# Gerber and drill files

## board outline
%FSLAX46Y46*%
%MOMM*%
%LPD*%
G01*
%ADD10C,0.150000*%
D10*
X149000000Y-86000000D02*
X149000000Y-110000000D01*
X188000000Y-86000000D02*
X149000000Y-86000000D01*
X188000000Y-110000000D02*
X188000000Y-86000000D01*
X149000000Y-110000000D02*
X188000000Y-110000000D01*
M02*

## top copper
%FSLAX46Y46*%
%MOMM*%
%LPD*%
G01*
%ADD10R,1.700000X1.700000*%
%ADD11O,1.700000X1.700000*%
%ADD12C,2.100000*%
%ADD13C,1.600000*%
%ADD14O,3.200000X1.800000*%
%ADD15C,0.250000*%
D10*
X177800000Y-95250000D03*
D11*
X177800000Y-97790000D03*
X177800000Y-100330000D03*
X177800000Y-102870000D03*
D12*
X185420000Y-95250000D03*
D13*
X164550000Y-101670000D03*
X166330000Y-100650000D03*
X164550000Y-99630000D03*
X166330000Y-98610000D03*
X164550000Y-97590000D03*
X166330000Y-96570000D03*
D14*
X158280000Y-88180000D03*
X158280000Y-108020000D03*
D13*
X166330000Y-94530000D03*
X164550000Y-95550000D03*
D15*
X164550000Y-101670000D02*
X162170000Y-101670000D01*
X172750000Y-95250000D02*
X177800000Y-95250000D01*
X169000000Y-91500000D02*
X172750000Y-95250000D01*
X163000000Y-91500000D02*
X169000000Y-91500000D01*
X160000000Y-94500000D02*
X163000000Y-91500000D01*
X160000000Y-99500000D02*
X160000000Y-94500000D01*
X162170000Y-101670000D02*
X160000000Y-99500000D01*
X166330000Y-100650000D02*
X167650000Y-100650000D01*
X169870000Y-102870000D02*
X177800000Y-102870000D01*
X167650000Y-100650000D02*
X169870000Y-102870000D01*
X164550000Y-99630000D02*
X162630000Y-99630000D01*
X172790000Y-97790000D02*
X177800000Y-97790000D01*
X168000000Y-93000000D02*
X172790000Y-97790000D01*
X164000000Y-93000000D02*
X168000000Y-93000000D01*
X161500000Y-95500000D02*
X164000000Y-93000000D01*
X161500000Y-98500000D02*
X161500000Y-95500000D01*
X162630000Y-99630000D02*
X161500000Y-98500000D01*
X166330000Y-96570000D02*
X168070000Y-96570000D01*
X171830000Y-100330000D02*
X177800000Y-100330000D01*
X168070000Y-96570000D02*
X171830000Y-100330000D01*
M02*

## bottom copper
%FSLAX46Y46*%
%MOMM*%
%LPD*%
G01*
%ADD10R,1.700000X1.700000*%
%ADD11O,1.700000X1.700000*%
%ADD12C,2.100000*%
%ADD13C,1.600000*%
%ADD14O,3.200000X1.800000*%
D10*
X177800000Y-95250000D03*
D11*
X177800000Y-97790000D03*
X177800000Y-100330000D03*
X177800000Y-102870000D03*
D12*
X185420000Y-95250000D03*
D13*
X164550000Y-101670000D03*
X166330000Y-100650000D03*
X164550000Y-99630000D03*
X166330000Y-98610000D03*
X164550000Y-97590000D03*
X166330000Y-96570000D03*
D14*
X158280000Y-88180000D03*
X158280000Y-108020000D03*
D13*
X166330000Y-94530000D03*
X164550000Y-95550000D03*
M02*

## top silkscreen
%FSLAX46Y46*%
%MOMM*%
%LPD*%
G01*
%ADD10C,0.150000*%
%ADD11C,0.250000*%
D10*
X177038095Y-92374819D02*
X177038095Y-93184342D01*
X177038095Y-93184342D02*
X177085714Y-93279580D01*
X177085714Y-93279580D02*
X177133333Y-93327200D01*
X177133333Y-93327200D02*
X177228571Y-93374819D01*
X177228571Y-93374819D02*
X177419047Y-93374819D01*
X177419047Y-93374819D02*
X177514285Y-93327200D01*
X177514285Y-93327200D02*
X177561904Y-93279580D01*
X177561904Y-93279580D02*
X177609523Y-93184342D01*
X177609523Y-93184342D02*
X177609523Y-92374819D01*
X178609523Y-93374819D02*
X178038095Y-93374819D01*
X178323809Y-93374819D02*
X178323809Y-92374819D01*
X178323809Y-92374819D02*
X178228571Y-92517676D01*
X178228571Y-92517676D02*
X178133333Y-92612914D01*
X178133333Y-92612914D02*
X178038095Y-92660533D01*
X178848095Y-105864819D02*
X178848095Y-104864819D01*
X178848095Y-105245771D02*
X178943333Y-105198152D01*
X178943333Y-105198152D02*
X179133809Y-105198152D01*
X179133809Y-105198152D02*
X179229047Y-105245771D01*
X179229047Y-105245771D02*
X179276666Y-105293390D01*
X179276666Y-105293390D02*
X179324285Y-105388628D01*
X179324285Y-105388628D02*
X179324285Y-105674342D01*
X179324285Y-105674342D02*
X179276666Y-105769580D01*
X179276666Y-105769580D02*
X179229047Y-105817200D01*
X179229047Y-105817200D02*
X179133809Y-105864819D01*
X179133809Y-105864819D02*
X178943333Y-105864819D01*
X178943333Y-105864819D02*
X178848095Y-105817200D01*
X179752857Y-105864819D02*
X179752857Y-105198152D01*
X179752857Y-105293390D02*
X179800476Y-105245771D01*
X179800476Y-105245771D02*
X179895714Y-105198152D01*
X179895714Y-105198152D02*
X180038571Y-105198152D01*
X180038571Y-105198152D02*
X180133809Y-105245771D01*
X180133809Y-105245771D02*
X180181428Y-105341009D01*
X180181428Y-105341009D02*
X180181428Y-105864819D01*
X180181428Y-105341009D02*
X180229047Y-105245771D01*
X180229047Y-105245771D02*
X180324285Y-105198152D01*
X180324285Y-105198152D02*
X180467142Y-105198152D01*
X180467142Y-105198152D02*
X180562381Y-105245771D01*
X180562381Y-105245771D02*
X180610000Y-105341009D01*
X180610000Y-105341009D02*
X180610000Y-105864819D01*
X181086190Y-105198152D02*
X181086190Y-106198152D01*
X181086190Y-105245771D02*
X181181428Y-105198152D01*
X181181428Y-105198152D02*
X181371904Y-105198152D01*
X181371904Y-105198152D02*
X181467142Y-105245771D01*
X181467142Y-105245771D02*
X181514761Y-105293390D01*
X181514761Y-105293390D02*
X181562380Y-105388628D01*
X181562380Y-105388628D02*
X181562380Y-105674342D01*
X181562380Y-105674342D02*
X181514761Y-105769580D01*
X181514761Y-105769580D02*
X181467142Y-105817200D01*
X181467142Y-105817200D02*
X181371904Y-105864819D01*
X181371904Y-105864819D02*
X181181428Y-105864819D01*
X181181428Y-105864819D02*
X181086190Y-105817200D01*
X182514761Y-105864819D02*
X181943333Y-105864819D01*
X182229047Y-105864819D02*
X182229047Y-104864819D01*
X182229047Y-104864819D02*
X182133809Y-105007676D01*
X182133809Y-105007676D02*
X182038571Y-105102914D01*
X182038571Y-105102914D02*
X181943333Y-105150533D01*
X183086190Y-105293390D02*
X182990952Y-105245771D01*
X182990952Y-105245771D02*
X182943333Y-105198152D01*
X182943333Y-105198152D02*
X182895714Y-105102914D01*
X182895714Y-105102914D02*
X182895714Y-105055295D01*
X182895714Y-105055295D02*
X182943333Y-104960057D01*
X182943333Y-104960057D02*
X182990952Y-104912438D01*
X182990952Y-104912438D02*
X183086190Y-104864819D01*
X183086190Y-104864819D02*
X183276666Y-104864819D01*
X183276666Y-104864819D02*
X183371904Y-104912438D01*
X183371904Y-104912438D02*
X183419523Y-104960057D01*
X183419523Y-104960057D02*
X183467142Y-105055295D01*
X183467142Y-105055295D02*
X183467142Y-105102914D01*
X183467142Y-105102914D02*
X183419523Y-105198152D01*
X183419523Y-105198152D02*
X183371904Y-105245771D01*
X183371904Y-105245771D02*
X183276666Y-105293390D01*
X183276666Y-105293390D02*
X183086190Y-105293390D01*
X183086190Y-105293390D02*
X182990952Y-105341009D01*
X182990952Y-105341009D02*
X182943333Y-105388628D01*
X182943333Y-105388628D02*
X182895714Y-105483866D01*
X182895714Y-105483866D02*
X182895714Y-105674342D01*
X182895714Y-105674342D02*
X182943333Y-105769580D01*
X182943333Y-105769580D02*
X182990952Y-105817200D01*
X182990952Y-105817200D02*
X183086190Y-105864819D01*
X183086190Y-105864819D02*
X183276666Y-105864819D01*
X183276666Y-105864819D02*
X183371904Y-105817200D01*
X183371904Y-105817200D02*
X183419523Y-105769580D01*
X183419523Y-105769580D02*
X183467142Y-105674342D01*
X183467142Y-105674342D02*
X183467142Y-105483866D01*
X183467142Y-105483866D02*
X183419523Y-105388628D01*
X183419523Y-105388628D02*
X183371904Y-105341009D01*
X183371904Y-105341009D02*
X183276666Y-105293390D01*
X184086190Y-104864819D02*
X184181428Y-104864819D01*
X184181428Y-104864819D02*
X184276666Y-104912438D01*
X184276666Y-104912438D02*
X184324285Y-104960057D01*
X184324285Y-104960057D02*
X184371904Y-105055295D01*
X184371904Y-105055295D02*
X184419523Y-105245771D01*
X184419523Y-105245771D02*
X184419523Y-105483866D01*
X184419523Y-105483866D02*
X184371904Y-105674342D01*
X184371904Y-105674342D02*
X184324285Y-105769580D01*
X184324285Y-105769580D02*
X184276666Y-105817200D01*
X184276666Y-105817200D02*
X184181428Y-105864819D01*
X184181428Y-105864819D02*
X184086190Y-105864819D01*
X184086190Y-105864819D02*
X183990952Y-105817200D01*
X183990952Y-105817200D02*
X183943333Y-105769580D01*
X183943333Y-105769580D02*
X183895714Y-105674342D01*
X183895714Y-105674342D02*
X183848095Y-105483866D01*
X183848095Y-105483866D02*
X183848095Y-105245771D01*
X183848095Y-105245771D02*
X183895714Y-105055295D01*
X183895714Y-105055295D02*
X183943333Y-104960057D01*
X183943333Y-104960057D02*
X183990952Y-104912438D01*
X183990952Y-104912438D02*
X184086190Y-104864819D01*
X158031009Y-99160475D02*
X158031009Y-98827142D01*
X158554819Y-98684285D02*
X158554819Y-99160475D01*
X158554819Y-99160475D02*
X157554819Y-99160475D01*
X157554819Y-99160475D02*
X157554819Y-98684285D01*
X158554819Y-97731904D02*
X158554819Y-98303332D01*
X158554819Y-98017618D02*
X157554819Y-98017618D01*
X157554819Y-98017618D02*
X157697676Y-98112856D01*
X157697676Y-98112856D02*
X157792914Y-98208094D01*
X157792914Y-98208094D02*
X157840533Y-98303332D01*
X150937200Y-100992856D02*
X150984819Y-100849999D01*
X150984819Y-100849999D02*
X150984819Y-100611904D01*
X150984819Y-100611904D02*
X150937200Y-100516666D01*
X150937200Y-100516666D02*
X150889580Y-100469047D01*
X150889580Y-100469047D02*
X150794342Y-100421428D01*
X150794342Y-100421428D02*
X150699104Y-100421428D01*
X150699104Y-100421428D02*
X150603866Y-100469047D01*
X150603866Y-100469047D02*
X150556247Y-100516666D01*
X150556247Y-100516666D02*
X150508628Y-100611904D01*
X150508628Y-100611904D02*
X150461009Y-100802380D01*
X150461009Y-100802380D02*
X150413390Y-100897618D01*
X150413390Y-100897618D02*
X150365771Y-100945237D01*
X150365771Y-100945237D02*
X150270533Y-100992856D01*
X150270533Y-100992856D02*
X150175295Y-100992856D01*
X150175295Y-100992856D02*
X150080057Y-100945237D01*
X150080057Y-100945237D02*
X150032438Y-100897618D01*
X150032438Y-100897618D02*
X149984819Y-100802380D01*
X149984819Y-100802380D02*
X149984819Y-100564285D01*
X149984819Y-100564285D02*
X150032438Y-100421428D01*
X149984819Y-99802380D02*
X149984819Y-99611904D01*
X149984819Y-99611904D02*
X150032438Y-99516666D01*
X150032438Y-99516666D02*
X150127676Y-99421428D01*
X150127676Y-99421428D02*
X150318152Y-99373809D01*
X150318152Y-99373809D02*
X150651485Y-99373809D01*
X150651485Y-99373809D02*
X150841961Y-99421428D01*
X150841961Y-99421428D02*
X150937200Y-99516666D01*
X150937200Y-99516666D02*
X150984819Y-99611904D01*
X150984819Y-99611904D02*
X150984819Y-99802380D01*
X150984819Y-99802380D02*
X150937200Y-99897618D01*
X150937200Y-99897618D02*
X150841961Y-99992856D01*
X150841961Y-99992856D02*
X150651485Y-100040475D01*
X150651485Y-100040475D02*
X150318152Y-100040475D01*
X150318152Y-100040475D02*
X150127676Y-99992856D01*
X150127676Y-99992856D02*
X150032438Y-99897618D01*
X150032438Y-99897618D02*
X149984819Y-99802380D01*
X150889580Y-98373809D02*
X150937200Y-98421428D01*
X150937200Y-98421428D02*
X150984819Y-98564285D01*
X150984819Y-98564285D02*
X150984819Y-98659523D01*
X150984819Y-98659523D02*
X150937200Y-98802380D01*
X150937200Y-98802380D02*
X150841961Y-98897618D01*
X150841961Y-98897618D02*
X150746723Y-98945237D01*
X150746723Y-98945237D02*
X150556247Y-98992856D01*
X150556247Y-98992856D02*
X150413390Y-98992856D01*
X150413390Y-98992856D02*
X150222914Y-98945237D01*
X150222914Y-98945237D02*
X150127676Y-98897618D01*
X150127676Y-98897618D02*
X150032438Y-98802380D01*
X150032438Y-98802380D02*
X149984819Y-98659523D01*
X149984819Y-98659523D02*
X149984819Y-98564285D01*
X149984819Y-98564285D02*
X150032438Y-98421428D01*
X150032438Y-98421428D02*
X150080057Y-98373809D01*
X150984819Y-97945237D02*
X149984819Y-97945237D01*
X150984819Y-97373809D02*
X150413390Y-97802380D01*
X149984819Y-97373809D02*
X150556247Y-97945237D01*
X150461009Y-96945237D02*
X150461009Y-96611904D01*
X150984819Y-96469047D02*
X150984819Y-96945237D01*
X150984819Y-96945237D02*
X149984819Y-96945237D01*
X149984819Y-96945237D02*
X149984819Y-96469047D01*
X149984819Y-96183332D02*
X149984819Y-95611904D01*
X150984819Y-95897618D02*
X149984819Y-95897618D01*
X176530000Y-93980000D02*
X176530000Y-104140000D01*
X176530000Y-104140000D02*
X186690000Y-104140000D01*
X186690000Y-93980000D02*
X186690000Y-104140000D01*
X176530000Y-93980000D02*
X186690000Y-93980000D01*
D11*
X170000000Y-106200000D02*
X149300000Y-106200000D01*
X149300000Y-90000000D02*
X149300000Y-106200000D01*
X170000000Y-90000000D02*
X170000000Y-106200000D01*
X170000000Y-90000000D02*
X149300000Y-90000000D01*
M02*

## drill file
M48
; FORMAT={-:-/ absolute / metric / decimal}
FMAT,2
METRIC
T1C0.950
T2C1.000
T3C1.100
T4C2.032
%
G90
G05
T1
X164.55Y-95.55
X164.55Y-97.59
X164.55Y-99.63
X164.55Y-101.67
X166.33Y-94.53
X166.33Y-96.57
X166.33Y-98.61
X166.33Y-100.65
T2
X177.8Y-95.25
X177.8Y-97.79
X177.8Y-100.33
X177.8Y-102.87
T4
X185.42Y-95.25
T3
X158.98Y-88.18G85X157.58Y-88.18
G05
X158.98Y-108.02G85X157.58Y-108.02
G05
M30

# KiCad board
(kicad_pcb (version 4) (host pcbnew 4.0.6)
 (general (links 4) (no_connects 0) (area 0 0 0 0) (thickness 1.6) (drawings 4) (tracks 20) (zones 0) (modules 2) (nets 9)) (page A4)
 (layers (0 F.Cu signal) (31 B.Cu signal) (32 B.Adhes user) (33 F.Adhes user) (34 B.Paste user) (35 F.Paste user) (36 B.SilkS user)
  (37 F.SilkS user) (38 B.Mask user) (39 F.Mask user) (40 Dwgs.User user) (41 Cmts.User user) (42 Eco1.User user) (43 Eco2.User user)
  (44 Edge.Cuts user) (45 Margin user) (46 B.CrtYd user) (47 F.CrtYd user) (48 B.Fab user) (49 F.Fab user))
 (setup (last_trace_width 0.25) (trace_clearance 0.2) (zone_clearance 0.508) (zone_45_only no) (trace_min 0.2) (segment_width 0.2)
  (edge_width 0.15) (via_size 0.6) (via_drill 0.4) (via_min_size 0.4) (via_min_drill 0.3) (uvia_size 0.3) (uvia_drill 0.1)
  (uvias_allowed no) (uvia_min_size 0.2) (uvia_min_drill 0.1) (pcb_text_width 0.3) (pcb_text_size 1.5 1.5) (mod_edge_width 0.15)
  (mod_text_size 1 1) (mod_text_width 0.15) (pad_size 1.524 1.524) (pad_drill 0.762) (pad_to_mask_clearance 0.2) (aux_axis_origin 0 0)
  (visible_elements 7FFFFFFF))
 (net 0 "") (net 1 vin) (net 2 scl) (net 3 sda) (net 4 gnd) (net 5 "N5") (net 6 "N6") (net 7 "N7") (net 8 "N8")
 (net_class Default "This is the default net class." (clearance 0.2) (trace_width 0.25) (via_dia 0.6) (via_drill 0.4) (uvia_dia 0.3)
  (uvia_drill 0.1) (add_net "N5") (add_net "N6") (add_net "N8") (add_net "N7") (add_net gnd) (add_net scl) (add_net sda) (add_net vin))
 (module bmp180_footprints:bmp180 (layer F.Cu) (at 177.8 95.25)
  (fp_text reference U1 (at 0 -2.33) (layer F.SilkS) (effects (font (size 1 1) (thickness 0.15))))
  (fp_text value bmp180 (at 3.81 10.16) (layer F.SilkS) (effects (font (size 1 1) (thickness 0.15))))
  (fp_line (start -1.27 -1.27) (end -1.27 8.89) (layer F.SilkS) (width 0.15))
  (fp_line (start -1.27 8.89) (end 8.89 8.89) (layer F.SilkS) (width 0.15))
  (fp_line (start 8.89 -1.27) (end 8.89 8.89) (layer F.SilkS) (width 0.15))
  (fp_line (start -1.27 -1.27) (end 8.89 -1.27) (layer F.SilkS) (width 0.15))
  (pad 1 thru_hole rect (at 0 0) (size 1.7 1.7) (drill 1) (layers *.Cu *.Mask) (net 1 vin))
  (pad 2 thru_hole oval (at 0 2.54) (size 1.7 1.7) (drill 1) (layers *.Cu *.Mask) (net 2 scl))
  (pad 3 thru_hole oval (at 0 5.08) (size 1.7 1.7) (drill 1) (layers *.Cu *.Mask) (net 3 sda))
  (pad 4 thru_hole oval (at 0 7.62) (size 1.7 1.7) (drill 1) (layers *.Cu *.Mask) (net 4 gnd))
  (pad "" np_thru_hole circle (at 7.62 0) (size 2.1 2.1) (drill 2.032) (layers *.Cu)))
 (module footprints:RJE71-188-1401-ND (layer F.Cu) (at 170 90 270)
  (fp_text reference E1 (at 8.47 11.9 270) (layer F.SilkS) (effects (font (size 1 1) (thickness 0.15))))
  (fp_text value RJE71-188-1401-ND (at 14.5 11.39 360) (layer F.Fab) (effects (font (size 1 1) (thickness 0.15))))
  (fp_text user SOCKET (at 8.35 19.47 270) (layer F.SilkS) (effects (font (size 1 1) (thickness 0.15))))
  (fp_line (start 16.2 0) (end 16.2 20.7) (layer F.SilkS) (width 0.25))
  (fp_line (start 0 20.7) (end 16.2 20.7) (layer F.SilkS) (width 0.25))
  (fp_line (start 0 0) (end 16.2 0) (layer F.SilkS) (width 0.25))
  (fp_line (start 0 0) (end 0 20.7) (layer F.SilkS) (width 0.25))
  (pad 1 thru_hole circle (at 11.67 5.45 270) (size 1.6 1.6) (drill 0.95) (layers *.Cu *.Mask) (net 1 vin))
  (pad 2 thru_hole circle (at 10.65 3.67 270) (size 1.6 1.6) (drill 0.95) (layers *.Cu *.Mask) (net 4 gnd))
  (pad 3 thru_hole circle (at 9.63 5.45 270) (size 1.6 1.6) (drill 0.95) (layers *.Cu *.Mask) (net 2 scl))
  (pad 4 thru_hole circle (at 8.61 3.67 270) (size 1.6 1.6) (drill 0.95) (layers *.Cu *.Mask) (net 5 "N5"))
  (pad 5 thru_hole circle (at 7.59 5.45 270) (size 1.6 1.6) (drill 0.95) (layers *.Cu *.Mask) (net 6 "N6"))
  (pad 6 thru_hole circle (at 6.57 3.67 270) (size 1.6 1.6) (drill 0.95) (layers *.Cu *.Mask) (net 3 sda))
  (pad "" thru_hole oval (at -1.82 11.72 270) (size 1.8 3.2) (drill oval 1.1 2.5) (layers *.Cu *.Mask))
  (pad "" thru_hole oval (at 18.02 11.72 270) (size 1.8 3.2) (drill oval 1.1 2.5) (layers *.Cu *.Mask))
  (pad 8 thru_hole circle (at 4.53 3.67 270) (size 1.6 1.6) (drill 0.95) (layers *.Cu *.Mask) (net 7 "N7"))
  (pad 7 thru_hole circle (at 5.55 5.45 270) (size 1.6 1.6) (drill 0.95) (layers *.Cu *.Mask) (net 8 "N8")))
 (gr_line (start 149 86) (end 149 110) (angle 90) (layer Edge.Cuts) (width 0.15))
 (gr_line (start 188 86) (end 149 86) (angle 90) (layer Edge.Cuts) (width 0.15))
 (gr_line (start 188 110) (end 188 86) (angle 90) (layer Edge.Cuts) (width 0.15))
 (gr_line (start 149 110) (end 188 110) (angle 90) (layer Edge.Cuts) (width 0.15))
 (segment (start 164.55 101.67) (end 162.17 101.67) (width 0.25) (layer F.Cu) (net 1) (status 400000))
 (segment (start 172.75 95.25) (end 177.8 95.25) (width 0.25) (layer F.Cu) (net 1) (status 800000))
 (segment (start 169 91.5) (end 172.75 95.25) (width 0.25) (layer F.Cu) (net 1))
 (segment (start 163 91.5) (end 169 91.5) (width 0.25) (layer F.Cu) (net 1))
 (segment (start 160 94.5) (end 163 91.5) (width 0.25) (layer F.Cu) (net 1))
 (segment (start 160 99.5) (end 160 94.5) (width 0.25) (layer F.Cu) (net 1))
 (segment (start 162.17 101.67) (end 160 99.5) (width 0.25) (layer F.Cu) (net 1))
 (segment (start 166.33 100.65) (end 167.65 100.65) (width 0.25) (layer F.Cu) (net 4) (status 400000))
 (segment (start 169.87 102.87) (end 177.8 102.87) (width 0.25) (layer F.Cu) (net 4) (status 800000))
 (segment (start 167.65 100.65) (end 169.87 102.87) (width 0.25) (layer F.Cu) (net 4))
 (segment (start 164.55 99.63) (end 162.63 99.63) (width 0.25) (layer F.Cu) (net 2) (status 400000))
 (segment (start 172.79 97.79) (end 177.8 97.79) (width 0.25) (layer F.Cu) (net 2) (status 800000))
 (segment (start 168 93) (end 172.79 97.79) (width 0.25) (layer F.Cu) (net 2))
 (segment (start 164 93) (end 168 93) (width 0.25) (layer F.Cu) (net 2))
 (segment (start 161.5 95.5) (end 164 93) (width 0.25) (layer F.Cu) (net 2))
 (segment (start 161.5 98.5) (end 161.5 95.5) (width 0.25) (layer F.Cu) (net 2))
 (segment (start 162.63 99.63) (end 161.5 98.5) (width 0.25) (layer F.Cu) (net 2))
 (segment (start 166.33 96.57) (end 168.07 96.57) (width 0.25) (layer F.Cu) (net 3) (status 400000))
 (segment (start 171.83 100.33) (end 177.8 100.33) (width 0.25) (layer F.Cu) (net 3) (status 800000))
 (segment (start 168.07 96.57) (end 171.83 100.33) (width 0.25) (layer F.Cu) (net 3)))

